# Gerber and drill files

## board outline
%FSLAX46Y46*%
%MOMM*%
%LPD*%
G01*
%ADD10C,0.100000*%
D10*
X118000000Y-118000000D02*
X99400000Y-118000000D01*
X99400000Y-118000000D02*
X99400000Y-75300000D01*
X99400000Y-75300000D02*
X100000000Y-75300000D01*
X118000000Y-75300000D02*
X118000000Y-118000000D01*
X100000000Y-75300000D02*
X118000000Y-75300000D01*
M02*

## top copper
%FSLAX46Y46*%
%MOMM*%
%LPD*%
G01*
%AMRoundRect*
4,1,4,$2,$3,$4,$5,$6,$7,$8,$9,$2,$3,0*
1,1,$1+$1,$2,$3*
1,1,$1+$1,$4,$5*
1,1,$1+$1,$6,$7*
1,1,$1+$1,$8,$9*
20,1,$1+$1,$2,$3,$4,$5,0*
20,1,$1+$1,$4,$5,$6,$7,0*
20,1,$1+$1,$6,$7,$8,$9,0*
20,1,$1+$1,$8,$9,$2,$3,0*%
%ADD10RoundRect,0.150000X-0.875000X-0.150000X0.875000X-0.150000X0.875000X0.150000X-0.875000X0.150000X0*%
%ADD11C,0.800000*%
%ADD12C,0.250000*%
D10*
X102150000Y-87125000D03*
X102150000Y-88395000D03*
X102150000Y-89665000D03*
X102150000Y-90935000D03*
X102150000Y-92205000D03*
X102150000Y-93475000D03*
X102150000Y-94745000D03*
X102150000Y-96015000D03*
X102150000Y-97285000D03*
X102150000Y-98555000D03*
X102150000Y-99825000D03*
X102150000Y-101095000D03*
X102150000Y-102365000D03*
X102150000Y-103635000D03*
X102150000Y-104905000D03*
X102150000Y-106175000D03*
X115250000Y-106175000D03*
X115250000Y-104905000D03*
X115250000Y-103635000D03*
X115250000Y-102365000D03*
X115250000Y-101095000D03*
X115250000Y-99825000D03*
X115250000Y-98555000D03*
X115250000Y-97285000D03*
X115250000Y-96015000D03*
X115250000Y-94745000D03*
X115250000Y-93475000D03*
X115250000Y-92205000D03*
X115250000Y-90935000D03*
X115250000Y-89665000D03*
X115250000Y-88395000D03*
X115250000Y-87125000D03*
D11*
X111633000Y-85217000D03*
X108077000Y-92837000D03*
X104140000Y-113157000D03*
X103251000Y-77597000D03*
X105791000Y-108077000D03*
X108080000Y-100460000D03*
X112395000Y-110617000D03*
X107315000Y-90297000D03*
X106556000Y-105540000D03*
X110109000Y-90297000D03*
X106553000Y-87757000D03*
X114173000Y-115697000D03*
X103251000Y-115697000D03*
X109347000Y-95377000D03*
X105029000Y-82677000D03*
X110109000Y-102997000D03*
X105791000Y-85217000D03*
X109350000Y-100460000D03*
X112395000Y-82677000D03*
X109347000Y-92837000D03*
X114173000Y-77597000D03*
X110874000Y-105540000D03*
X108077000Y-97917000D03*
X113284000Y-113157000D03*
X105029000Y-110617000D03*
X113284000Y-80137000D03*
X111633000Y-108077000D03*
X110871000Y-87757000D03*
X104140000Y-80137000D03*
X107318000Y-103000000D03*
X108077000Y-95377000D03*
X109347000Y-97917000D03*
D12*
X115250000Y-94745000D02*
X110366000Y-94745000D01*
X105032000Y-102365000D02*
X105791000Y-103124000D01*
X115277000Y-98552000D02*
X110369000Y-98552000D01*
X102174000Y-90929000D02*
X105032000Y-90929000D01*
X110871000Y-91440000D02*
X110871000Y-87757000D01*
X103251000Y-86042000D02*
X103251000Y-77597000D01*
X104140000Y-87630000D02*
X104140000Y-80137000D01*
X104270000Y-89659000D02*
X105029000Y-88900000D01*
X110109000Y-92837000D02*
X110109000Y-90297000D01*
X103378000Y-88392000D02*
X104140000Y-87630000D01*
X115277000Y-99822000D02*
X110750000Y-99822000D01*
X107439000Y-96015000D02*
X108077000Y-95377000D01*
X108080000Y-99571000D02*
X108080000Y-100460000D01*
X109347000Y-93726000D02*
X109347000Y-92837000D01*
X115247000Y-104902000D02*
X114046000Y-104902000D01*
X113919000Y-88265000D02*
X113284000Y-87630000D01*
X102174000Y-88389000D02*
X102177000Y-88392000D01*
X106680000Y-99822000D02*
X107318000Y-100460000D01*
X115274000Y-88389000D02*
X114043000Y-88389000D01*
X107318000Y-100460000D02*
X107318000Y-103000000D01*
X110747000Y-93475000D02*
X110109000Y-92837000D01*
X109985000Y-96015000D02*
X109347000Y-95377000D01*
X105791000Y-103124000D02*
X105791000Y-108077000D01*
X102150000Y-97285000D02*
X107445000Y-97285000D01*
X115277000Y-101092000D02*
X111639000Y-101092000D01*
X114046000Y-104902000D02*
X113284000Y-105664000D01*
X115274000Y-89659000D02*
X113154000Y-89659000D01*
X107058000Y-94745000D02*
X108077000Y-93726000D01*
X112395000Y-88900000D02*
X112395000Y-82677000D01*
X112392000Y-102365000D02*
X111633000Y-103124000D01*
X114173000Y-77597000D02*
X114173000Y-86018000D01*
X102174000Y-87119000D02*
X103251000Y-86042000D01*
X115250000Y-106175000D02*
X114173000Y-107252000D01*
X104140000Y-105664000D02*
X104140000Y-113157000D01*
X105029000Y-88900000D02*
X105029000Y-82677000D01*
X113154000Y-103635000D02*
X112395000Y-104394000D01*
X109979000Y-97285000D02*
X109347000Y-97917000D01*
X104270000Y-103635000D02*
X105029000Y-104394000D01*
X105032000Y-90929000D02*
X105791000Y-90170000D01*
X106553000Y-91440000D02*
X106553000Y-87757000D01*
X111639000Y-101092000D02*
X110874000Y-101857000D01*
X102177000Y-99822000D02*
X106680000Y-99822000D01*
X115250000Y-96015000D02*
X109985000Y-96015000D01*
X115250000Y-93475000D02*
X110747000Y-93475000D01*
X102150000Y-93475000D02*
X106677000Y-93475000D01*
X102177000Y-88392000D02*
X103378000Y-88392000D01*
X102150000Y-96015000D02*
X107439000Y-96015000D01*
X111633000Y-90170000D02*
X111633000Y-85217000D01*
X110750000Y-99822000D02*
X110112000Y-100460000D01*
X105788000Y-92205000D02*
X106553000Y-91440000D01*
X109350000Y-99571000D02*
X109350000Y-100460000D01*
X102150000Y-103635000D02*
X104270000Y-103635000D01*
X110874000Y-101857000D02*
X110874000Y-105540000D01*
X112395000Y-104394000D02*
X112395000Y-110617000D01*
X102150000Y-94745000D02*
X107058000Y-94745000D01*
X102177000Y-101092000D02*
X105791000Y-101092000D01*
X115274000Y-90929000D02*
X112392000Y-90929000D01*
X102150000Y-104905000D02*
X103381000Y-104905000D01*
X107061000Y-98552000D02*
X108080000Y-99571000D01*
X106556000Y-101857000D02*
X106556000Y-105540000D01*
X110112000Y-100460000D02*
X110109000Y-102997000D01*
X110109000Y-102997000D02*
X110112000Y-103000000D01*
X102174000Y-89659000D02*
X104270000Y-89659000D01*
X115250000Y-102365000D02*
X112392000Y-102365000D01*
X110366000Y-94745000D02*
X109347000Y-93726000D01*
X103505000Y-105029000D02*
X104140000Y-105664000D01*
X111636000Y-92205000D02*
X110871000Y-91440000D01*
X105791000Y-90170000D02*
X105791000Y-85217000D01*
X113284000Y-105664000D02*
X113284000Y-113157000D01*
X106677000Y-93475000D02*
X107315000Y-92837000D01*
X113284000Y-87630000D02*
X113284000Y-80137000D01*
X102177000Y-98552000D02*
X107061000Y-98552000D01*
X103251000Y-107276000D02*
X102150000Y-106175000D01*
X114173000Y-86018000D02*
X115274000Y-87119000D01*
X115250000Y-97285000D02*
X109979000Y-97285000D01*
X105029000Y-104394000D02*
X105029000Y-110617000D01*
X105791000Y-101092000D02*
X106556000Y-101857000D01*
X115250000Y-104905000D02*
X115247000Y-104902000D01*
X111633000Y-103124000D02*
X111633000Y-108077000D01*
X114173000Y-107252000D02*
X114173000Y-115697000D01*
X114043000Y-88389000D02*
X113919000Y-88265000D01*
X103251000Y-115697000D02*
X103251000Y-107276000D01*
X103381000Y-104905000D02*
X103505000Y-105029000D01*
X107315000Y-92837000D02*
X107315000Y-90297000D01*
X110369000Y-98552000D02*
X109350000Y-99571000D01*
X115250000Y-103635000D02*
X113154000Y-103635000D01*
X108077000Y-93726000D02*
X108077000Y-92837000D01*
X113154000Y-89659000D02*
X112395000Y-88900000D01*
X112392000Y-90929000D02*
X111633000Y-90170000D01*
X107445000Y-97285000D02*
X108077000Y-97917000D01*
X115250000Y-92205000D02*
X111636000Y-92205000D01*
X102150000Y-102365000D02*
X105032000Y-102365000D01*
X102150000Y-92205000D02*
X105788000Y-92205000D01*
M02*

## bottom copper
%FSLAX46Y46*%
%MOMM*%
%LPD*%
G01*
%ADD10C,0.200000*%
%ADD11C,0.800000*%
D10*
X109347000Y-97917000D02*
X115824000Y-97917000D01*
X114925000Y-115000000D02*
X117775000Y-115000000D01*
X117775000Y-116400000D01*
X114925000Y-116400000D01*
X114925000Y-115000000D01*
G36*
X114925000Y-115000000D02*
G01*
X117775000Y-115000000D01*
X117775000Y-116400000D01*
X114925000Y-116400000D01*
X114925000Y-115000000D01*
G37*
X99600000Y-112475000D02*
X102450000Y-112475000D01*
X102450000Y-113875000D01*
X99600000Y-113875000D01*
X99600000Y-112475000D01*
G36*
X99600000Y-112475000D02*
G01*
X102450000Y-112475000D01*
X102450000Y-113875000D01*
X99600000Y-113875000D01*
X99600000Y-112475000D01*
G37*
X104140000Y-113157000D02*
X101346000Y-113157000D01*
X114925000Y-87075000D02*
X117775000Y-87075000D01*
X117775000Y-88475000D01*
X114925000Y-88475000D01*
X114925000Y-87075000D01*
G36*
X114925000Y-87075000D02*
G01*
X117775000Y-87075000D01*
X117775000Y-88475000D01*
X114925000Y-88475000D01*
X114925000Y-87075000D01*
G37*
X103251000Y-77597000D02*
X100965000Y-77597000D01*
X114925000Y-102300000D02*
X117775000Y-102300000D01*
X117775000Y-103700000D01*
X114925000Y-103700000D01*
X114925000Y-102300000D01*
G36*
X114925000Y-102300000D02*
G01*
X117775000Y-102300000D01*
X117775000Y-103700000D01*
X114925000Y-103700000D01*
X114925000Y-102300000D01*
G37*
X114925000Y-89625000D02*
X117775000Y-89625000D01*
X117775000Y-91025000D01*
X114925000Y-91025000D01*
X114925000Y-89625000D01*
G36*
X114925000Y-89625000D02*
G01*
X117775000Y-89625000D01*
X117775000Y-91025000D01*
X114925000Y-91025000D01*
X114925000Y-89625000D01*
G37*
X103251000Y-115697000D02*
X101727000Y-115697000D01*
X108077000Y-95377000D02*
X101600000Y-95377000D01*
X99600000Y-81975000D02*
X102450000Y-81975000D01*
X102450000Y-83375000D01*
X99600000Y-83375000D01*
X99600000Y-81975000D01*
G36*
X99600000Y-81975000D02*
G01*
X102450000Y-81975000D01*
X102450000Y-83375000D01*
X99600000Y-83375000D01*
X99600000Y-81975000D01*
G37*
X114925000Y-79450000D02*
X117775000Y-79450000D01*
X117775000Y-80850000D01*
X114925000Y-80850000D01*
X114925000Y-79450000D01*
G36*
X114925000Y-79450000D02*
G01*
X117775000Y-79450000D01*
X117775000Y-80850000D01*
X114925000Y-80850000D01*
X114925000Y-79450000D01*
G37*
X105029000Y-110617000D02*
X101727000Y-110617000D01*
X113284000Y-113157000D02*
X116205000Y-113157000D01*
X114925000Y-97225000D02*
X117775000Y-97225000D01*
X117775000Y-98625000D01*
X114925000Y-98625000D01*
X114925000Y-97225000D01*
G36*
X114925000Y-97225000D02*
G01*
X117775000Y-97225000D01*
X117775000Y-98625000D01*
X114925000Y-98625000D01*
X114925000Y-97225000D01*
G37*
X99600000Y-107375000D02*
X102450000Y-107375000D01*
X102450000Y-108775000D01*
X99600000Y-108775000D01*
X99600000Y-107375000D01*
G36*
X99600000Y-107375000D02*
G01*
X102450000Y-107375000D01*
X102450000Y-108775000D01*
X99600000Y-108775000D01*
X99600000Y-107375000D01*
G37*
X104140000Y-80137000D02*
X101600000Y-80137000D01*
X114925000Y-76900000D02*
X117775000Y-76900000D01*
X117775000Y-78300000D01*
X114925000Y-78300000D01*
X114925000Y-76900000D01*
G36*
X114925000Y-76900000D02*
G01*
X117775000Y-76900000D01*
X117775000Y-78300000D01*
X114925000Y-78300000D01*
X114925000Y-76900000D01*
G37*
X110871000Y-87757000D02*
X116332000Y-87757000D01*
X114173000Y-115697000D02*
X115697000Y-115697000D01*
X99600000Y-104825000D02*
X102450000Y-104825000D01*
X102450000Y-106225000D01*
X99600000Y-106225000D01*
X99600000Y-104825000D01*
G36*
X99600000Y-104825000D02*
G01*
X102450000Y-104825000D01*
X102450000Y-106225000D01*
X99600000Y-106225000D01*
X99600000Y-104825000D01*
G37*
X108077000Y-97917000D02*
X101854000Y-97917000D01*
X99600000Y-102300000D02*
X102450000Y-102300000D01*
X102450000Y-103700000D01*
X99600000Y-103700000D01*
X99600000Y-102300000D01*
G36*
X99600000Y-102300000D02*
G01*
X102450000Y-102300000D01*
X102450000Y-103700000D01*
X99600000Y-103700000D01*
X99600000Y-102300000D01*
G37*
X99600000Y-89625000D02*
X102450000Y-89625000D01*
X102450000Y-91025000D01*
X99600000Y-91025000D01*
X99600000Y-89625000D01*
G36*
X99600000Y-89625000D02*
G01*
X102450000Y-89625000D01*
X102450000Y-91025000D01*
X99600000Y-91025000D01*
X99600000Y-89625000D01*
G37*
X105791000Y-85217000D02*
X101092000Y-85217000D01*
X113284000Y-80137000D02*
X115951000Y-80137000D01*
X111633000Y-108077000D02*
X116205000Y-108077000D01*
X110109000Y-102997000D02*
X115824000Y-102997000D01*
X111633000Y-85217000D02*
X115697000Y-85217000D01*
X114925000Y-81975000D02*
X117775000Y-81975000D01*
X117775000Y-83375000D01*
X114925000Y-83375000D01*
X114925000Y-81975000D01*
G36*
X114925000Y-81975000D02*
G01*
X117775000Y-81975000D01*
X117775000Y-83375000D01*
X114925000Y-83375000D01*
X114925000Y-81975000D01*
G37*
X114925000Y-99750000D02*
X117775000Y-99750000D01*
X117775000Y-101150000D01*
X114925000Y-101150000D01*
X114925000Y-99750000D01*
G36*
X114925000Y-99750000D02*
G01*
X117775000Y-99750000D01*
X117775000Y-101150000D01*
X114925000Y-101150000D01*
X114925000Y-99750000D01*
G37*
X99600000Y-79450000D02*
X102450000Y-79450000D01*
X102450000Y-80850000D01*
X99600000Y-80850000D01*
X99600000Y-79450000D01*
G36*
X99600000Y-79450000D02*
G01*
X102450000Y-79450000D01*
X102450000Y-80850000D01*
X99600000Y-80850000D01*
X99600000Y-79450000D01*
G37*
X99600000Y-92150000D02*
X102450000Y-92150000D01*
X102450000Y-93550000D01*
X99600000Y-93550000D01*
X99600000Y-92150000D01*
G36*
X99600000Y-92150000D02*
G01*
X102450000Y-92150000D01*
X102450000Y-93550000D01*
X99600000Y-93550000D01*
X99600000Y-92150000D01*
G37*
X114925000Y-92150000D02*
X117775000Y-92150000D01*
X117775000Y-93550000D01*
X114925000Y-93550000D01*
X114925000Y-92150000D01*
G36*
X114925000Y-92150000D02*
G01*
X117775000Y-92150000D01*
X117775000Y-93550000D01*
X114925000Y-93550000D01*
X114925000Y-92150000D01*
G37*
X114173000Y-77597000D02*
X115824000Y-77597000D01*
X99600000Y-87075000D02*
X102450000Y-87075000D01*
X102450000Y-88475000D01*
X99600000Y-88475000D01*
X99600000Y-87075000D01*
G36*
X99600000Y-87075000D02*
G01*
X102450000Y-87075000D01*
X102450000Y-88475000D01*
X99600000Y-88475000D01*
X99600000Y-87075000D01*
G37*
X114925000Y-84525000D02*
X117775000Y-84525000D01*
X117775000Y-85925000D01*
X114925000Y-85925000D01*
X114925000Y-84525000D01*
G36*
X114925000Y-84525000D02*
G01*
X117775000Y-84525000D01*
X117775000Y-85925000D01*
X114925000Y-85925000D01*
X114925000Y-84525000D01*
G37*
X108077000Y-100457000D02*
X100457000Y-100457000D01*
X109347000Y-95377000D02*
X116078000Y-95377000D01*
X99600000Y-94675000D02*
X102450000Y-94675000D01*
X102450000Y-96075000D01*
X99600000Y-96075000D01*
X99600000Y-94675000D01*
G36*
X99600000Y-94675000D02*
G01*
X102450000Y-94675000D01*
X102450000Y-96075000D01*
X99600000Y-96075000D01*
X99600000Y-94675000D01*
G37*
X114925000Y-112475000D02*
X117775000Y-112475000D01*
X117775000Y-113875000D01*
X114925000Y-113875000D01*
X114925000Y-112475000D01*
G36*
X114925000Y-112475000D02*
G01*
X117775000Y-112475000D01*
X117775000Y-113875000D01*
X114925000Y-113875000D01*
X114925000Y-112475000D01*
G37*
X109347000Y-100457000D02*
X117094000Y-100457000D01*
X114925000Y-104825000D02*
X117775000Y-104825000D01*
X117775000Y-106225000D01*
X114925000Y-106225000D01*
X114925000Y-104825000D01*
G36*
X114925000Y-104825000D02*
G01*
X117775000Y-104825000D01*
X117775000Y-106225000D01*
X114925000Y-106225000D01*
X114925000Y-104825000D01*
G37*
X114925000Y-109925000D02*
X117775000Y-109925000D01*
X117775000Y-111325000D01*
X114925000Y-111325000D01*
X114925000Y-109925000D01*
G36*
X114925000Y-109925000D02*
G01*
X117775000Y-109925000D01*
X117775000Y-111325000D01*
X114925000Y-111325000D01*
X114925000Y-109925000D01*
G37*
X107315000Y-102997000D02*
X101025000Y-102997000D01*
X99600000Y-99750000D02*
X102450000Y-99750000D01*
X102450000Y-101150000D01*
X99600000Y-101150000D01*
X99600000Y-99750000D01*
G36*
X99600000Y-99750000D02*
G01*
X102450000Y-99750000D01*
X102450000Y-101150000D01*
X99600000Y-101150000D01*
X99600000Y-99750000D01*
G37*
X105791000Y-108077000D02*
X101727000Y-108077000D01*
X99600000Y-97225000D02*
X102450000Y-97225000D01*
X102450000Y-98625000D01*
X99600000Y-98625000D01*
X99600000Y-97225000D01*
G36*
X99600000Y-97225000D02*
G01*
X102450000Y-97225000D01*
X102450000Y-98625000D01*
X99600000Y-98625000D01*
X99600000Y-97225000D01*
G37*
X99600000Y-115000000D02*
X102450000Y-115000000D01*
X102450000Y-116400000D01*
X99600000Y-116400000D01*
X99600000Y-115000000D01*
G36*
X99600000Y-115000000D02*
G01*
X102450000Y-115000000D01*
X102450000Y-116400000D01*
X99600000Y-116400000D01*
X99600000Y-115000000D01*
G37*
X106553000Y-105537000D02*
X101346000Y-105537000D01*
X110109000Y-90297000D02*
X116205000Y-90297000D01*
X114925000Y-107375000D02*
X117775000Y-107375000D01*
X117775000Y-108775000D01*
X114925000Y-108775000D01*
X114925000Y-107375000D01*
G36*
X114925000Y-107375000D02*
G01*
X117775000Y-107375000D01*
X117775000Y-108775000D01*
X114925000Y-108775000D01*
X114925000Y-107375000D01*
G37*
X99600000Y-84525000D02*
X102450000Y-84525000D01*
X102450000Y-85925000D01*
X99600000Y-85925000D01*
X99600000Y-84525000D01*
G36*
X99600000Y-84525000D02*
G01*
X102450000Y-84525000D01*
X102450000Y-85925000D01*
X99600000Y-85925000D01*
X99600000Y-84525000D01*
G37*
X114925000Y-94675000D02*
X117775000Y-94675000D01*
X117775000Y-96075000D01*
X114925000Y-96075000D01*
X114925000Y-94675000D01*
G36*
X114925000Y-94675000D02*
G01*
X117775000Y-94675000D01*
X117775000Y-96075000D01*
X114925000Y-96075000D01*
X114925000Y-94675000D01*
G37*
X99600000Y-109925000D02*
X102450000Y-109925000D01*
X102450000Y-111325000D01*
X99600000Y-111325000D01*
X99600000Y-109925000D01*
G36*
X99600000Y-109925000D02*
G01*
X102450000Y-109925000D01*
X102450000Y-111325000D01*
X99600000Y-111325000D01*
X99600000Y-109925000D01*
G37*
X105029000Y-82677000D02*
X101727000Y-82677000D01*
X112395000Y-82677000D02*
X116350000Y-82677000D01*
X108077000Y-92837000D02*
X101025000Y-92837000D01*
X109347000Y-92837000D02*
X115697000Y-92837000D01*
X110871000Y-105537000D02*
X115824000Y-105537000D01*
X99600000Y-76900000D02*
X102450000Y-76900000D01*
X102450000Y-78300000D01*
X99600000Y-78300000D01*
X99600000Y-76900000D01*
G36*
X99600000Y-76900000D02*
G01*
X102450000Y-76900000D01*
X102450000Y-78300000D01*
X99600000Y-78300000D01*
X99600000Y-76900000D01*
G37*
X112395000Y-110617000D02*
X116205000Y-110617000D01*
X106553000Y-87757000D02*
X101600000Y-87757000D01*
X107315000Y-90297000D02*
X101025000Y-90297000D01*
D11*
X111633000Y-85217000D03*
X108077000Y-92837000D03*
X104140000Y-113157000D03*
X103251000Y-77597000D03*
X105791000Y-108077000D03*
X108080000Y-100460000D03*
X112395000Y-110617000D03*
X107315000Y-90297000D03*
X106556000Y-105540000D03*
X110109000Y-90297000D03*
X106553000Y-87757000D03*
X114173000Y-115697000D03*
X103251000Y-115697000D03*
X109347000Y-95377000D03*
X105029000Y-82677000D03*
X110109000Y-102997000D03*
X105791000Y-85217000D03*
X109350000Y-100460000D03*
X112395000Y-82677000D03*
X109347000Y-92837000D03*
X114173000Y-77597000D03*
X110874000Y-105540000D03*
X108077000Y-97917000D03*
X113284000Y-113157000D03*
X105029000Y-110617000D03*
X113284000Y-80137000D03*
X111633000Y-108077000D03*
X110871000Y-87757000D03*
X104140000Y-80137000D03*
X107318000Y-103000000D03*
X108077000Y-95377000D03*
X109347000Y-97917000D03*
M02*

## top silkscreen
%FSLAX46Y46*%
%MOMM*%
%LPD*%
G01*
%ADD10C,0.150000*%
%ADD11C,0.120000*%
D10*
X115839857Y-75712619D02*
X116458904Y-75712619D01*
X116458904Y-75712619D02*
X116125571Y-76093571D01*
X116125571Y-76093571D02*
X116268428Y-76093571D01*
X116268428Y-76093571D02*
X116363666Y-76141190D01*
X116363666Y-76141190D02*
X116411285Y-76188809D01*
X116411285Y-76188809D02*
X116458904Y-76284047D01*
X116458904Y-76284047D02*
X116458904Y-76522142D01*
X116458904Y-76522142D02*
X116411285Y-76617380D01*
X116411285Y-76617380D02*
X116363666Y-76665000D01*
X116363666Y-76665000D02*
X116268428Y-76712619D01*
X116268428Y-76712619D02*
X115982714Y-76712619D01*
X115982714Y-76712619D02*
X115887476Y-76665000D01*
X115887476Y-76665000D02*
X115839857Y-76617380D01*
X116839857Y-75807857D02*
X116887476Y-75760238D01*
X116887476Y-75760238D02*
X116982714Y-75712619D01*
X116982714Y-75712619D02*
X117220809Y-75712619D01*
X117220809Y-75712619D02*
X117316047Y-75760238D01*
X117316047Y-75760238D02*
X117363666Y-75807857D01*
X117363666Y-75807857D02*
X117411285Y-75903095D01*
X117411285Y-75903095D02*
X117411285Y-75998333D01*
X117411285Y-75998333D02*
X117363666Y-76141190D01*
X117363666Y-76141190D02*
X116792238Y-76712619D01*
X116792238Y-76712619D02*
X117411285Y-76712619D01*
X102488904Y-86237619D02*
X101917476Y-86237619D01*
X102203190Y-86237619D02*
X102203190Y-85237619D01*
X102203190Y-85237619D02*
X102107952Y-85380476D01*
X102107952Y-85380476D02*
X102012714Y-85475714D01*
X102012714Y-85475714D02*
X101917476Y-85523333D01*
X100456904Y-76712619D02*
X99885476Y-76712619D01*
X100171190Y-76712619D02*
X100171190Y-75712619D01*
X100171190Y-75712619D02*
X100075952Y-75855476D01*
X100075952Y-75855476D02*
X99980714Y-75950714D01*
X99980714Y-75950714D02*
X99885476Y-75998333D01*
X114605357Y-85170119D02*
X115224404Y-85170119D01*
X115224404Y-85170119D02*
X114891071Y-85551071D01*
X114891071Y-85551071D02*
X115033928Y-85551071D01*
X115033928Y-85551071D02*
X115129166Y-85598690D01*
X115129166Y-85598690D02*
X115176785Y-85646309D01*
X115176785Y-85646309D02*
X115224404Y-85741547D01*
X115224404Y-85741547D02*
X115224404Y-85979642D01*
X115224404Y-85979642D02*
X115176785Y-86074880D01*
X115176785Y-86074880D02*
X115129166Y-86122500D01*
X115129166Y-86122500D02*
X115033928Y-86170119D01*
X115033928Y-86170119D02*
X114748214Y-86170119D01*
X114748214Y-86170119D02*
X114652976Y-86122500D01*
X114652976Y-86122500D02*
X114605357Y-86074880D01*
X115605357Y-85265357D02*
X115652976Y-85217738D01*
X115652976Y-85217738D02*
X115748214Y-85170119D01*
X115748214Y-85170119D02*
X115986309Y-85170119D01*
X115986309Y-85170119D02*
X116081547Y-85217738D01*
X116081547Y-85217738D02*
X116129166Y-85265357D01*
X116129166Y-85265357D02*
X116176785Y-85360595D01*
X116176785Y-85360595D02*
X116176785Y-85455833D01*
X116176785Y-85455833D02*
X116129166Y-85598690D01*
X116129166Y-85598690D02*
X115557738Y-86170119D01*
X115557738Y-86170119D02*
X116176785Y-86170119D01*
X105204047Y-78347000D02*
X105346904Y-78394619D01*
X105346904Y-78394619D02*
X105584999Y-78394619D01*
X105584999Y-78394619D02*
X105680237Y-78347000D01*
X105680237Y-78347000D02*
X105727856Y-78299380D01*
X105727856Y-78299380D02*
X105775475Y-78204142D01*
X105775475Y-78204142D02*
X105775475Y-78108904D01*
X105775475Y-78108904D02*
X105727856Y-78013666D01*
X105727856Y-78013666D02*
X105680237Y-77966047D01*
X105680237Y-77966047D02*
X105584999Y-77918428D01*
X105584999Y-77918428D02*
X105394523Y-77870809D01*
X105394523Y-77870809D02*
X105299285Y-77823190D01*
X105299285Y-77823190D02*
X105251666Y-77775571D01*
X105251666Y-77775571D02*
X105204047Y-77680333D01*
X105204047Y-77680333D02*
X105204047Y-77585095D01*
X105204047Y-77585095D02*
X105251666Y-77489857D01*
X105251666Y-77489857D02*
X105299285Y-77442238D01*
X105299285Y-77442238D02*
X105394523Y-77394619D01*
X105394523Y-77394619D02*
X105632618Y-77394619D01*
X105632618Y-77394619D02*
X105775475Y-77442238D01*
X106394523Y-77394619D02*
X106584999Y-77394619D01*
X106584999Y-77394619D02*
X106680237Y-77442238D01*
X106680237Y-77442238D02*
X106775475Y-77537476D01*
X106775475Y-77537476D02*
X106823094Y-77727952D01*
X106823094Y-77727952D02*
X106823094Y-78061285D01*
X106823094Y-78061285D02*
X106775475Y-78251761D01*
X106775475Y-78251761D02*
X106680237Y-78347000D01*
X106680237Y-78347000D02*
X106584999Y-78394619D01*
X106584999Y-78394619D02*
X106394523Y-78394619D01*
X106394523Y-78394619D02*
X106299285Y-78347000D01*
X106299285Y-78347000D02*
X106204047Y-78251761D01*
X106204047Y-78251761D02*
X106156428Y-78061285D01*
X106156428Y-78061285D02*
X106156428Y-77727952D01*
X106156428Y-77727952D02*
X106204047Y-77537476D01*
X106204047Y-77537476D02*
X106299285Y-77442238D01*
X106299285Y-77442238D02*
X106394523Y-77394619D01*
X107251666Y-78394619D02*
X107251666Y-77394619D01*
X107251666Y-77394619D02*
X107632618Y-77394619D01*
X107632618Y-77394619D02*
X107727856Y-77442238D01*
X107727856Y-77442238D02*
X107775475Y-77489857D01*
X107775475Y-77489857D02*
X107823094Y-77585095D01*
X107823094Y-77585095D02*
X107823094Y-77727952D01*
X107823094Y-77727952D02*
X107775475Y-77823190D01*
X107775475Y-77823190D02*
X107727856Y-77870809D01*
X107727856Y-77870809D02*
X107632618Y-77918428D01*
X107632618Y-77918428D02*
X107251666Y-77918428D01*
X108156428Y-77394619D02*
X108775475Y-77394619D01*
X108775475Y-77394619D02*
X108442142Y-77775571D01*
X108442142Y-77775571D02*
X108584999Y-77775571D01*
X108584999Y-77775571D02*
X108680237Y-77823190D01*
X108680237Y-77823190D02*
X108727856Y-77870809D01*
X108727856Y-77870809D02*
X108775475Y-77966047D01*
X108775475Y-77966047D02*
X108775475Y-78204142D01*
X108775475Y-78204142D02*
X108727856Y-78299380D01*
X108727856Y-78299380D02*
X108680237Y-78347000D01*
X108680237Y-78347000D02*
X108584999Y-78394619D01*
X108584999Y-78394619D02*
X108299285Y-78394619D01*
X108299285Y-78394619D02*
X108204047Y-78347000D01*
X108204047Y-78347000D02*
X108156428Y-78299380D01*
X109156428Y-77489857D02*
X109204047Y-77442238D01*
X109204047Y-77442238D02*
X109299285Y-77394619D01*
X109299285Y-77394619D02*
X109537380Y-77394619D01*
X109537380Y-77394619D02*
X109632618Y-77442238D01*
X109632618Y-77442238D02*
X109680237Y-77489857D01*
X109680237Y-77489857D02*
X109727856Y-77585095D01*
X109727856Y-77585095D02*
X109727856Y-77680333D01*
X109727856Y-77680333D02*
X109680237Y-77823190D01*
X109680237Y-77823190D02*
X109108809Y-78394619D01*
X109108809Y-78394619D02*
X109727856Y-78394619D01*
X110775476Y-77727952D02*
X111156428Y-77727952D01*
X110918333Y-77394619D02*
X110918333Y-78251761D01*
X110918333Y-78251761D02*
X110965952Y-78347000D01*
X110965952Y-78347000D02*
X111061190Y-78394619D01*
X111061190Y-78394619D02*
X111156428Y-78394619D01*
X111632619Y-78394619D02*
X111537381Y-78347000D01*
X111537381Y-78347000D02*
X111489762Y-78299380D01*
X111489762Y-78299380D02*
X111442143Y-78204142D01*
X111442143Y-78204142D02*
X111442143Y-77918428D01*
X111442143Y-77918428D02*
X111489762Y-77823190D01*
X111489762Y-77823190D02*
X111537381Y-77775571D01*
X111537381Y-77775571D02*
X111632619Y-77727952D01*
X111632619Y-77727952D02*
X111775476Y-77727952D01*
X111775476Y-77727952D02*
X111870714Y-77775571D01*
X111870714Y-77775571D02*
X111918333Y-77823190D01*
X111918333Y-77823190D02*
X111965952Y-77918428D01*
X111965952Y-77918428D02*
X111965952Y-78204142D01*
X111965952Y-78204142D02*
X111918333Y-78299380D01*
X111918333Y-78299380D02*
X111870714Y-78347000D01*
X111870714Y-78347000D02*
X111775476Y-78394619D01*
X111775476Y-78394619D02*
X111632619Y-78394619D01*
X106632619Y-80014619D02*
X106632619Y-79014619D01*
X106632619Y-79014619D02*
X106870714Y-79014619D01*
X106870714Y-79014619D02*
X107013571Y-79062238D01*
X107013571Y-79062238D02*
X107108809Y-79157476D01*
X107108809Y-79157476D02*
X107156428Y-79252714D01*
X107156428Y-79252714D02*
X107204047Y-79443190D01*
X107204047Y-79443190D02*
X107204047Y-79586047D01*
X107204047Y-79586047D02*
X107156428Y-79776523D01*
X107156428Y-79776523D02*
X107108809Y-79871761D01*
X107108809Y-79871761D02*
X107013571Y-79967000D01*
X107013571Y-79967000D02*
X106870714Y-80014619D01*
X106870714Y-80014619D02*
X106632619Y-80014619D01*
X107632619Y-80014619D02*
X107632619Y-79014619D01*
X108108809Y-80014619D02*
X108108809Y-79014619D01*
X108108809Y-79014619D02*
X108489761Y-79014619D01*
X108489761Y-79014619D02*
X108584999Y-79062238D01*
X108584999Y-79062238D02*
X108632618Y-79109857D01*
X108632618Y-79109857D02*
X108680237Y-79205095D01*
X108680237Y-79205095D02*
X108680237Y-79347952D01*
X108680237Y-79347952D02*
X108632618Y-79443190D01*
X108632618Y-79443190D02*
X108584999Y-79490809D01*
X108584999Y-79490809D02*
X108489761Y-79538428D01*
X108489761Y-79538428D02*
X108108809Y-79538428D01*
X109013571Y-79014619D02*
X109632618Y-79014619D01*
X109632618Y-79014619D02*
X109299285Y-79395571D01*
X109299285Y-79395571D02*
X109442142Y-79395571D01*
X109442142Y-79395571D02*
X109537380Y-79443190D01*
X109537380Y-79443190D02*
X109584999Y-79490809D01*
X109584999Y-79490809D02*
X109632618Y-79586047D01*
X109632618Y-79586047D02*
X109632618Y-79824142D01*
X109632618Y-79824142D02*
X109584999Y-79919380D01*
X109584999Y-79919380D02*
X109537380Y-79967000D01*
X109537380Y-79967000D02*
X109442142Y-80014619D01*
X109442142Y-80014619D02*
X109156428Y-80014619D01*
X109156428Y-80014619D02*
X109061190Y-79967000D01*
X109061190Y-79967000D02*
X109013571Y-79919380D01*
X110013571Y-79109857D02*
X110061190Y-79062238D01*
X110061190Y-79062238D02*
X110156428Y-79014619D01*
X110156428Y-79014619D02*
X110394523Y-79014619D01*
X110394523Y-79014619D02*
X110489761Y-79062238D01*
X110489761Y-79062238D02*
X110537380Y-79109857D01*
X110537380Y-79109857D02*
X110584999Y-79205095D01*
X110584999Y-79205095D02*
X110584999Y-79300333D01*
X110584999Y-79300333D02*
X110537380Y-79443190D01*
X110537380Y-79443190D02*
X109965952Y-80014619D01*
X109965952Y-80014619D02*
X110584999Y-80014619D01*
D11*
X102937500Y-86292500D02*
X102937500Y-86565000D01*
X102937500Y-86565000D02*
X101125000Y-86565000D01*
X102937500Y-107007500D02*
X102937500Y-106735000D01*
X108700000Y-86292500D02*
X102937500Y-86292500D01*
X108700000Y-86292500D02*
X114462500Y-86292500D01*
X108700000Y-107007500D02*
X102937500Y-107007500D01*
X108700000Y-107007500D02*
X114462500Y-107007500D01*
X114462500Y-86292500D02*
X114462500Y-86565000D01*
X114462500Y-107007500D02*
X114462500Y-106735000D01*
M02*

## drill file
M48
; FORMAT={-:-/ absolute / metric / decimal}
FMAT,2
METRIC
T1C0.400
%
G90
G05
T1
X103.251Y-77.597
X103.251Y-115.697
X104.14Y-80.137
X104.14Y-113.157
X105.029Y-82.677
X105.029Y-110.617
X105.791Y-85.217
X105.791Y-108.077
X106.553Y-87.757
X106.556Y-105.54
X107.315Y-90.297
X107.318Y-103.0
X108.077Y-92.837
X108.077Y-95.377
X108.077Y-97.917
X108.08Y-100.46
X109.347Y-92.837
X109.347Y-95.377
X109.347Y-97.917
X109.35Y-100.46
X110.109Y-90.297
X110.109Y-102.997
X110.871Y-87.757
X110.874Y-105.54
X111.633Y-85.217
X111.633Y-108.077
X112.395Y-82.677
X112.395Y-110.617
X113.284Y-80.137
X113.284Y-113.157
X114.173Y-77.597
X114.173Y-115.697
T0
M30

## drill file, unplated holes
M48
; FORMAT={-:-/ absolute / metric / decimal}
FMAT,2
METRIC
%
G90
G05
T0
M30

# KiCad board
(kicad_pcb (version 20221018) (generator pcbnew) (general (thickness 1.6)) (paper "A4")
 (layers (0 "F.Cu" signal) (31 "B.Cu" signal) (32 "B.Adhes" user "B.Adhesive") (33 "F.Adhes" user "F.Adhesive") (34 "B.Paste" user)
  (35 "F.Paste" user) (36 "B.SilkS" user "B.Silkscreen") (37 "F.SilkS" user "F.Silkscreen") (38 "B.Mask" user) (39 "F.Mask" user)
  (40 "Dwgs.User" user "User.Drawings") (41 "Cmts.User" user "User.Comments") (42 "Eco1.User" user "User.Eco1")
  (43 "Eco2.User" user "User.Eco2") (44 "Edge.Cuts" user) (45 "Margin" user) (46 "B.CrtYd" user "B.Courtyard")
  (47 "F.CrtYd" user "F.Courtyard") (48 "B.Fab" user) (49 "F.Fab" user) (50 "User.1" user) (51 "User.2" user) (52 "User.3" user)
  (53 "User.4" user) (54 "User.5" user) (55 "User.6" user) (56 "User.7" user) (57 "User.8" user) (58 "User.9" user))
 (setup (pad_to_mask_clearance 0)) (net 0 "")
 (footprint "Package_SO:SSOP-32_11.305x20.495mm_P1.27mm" (layer "F.Cu") (at 108.7 96.65)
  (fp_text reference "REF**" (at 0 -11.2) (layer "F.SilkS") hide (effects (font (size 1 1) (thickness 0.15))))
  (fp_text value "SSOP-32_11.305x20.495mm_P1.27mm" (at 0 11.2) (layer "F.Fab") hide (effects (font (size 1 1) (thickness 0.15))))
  (fp_line (start -5.7625 -10.3575) (end -5.7625 -10.085) (stroke (width 0.12) (type solid)) (layer "F.SilkS"))
  (fp_line (start -5.7625 -10.085) (end -7.575 -10.085) (stroke (width 0.12) (type solid)) (layer "F.SilkS"))
  (fp_line (start -5.7625 10.3575) (end -5.7625 10.085) (stroke (width 0.12) (type solid)) (layer "F.SilkS"))
  (fp_line (start 0 -10.3575) (end -5.7625 -10.3575) (stroke (width 0.12) (type solid)) (layer "F.SilkS"))
  (fp_line (start 0 -10.3575) (end 5.7625 -10.3575) (stroke (width 0.12) (type solid)) (layer "F.SilkS"))
  (fp_line (start 0 10.3575) (end -5.7625 10.3575) (stroke (width 0.12) (type solid)) (layer "F.SilkS"))
  (fp_line (start 0 10.3575) (end 5.7625 10.3575) (stroke (width 0.12) (type solid)) (layer "F.SilkS"))
  (fp_line (start 5.7625 -10.3575) (end 5.7625 -10.085) (stroke (width 0.12) (type solid)) (layer "F.SilkS"))
  (fp_line (start 5.7625 10.3575) (end 5.7625 10.085) (stroke (width 0.12) (type solid)) (layer "F.SilkS"))
  (pad "1" smd roundrect (at -6.55 -9.525) (size 2.05 0.6) (layers "F.Cu" "F.Paste" "F.Mask") (roundrect_rratio 0.25))
  (pad "2" smd roundrect (at -6.55 -8.255) (size 2.05 0.6) (layers "F.Cu" "F.Paste" "F.Mask") (roundrect_rratio 0.25))
  (pad "3" smd roundrect (at -6.55 -6.985) (size 2.05 0.6) (layers "F.Cu" "F.Paste" "F.Mask") (roundrect_rratio 0.25))
  (pad "4" smd roundrect (at -6.55 -5.715) (size 2.05 0.6) (layers "F.Cu" "F.Paste" "F.Mask") (roundrect_rratio 0.25))
  (pad "5" smd roundrect (at -6.55 -4.445) (size 2.05 0.6) (layers "F.Cu" "F.Paste" "F.Mask") (roundrect_rratio 0.25))
  (pad "6" smd roundrect (at -6.55 -3.175) (size 2.05 0.6) (layers "F.Cu" "F.Paste" "F.Mask") (roundrect_rratio 0.25))
  (pad "7" smd roundrect (at -6.55 -1.905) (size 2.05 0.6) (layers "F.Cu" "F.Paste" "F.Mask") (roundrect_rratio 0.25))
  (pad "8" smd roundrect (at -6.55 -0.635) (size 2.05 0.6) (layers "F.Cu" "F.Paste" "F.Mask") (roundrect_rratio 0.25))
  (pad "9" smd roundrect (at -6.55 0.635) (size 2.05 0.6) (layers "F.Cu" "F.Paste" "F.Mask") (roundrect_rratio 0.25))
  (pad "10" smd roundrect (at -6.55 1.905) (size 2.05 0.6) (layers "F.Cu" "F.Paste" "F.Mask") (roundrect_rratio 0.25))
  (pad "11" smd roundrect (at -6.55 3.175) (size 2.05 0.6) (layers "F.Cu" "F.Paste" "F.Mask") (roundrect_rratio 0.25))
  (pad "12" smd roundrect (at -6.55 4.445) (size 2.05 0.6) (layers "F.Cu" "F.Paste" "F.Mask") (roundrect_rratio 0.25))
  (pad "13" smd roundrect (at -6.55 5.715) (size 2.05 0.6) (layers "F.Cu" "F.Paste" "F.Mask") (roundrect_rratio 0.25))
  (pad "14" smd roundrect (at -6.55 6.985) (size 2.05 0.6) (layers "F.Cu" "F.Paste" "F.Mask") (roundrect_rratio 0.25))
  (pad "15" smd roundrect (at -6.55 8.255) (size 2.05 0.6) (layers "F.Cu" "F.Paste" "F.Mask") (roundrect_rratio 0.25))
  (pad "16" smd roundrect (at -6.55 9.525) (size 2.05 0.6) (layers "F.Cu" "F.Paste" "F.Mask") (roundrect_rratio 0.25))
  (pad "17" smd roundrect (at 6.55 9.525) (size 2.05 0.6) (layers "F.Cu" "F.Paste" "F.Mask") (roundrect_rratio 0.25))
  (pad "18" smd roundrect (at 6.55 8.255) (size 2.05 0.6) (layers "F.Cu" "F.Paste" "F.Mask") (roundrect_rratio 0.25))
  (pad "19" smd roundrect (at 6.55 6.985) (size 2.05 0.6) (layers "F.Cu" "F.Paste" "F.Mask") (roundrect_rratio 0.25))
  (pad "20" smd roundrect (at 6.55 5.715) (size 2.05 0.6) (layers "F.Cu" "F.Paste" "F.Mask") (roundrect_rratio 0.25))
  (pad "21" smd roundrect (at 6.55 4.445) (size 2.05 0.6) (layers "F.Cu" "F.Paste" "F.Mask") (roundrect_rratio 0.25))
  (pad "22" smd roundrect (at 6.55 3.175) (size 2.05 0.6) (layers "F.Cu" "F.Paste" "F.Mask") (roundrect_rratio 0.25))
  (pad "23" smd roundrect (at 6.55 1.905) (size 2.05 0.6) (layers "F.Cu" "F.Paste" "F.Mask") (roundrect_rratio 0.25))
  (pad "24" smd roundrect (at 6.55 0.635) (size 2.05 0.6) (layers "F.Cu" "F.Paste" "F.Mask") (roundrect_rratio 0.25))
  (pad "25" smd roundrect (at 6.55 -0.635) (size 2.05 0.6) (layers "F.Cu" "F.Paste" "F.Mask") (roundrect_rratio 0.25))
  (pad "26" smd roundrect (at 6.55 -1.905) (size 2.05 0.6) (layers "F.Cu" "F.Paste" "F.Mask") (roundrect_rratio 0.25))
  (pad "27" smd roundrect (at 6.55 -3.175) (size 2.05 0.6) (layers "F.Cu" "F.Paste" "F.Mask") (roundrect_rratio 0.25))
  (pad "28" smd roundrect (at 6.55 -4.445) (size 2.05 0.6) (layers "F.Cu" "F.Paste" "F.Mask") (roundrect_rratio 0.25))
  (pad "29" smd roundrect (at 6.55 -5.715) (size 2.05 0.6) (layers "F.Cu" "F.Paste" "F.Mask") (roundrect_rratio 0.25))
  (pad "30" smd roundrect (at 6.55 -6.985) (size 2.05 0.6) (layers "F.Cu" "F.Paste" "F.Mask") (roundrect_rratio 0.25))
  (pad "31" smd roundrect (at 6.55 -8.255) (size 2.05 0.6) (layers "F.Cu" "F.Paste" "F.Mask") (roundrect_rratio 0.25))
  (pad "32" smd roundrect (at 6.55 -9.525) (size 2.05 0.6) (layers "F.Cu" "F.Paste" "F.Mask") (roundrect_rratio 0.25)))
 (gr_line (start 109.347 97.917) (end 115.824 97.917) (stroke (width 0.2) (type default)) (layer "B.Cu"))
 (gr_rect (start 114.925 115) (end 117.775 116.4) (stroke (width 0.2) (type solid)) (fill solid) (layer "B.Cu"))
 (gr_rect (start 99.6 112.475) (end 102.45 113.875) (stroke (width 0.2) (type solid)) (fill solid) (layer "B.Cu"))
 (gr_line (start 104.14 113.157) (end 101.346 113.157) (stroke (width 0.2) (type default)) (layer "B.Cu"))
 (gr_rect (start 114.925 87.075) (end 117.775 88.475) (stroke (width 0.2) (type solid)) (fill solid) (layer "B.Cu"))
 (gr_line (start 103.251 77.597) (end 100.965 77.597) (stroke (width 0.2) (type default)) (layer "B.Cu"))
 (gr_rect (start 114.925 102.3) (end 117.775 103.7) (stroke (width 0.2) (type solid)) (fill solid) (layer "B.Cu"))
 (gr_rect (start 114.925 89.625) (end 117.775 91.025) (stroke (width 0.2) (type solid)) (fill solid) (layer "B.Cu"))
 (gr_line (start 103.251 115.697) (end 101.727 115.697) (stroke (width 0.2) (type default)) (layer "B.Cu"))
 (gr_line (start 108.077 95.377) (end 101.6 95.377) (stroke (width 0.2) (type default)) (layer "B.Cu"))
 (gr_rect (start 99.6 81.975) (end 102.45 83.375) (stroke (width 0.2) (type solid)) (fill solid) (layer "B.Cu"))
 (gr_rect (start 114.925 79.45) (end 117.775 80.85) (stroke (width 0.2) (type solid)) (fill solid) (layer "B.Cu"))
 (gr_line (start 105.029 110.617) (end 101.727 110.617) (stroke (width 0.2) (type default)) (layer "B.Cu"))
 (gr_line (start 113.284 113.157) (end 116.205 113.157) (stroke (width 0.2) (type default)) (layer "B.Cu"))
 (gr_rect (start 114.925 97.225) (end 117.775 98.625) (stroke (width 0.2) (type solid)) (fill solid) (layer "B.Cu"))
 (gr_rect (start 99.6 107.375) (end 102.45 108.775) (stroke (width 0.2) (type solid)) (fill solid) (layer "B.Cu"))
 (gr_line (start 104.14 80.137) (end 101.6 80.137) (stroke (width 0.2) (type default)) (layer "B.Cu"))
 (gr_rect (start 114.925 76.9) (end 117.775 78.3) (stroke (width 0.2) (type solid)) (fill solid) (layer "B.Cu"))
 (gr_line (start 110.871 87.757) (end 116.332 87.757) (stroke (width 0.2) (type default)) (layer "B.Cu"))
 (gr_line (start 114.173 115.697) (end 115.697 115.697) (stroke (width 0.2) (type default)) (layer "B.Cu"))
 (gr_rect (start 99.6 104.825) (end 102.45 106.225) (stroke (width 0.2) (type solid)) (fill solid) (layer "B.Cu"))
 (gr_line (start 108.077 97.917) (end 101.854 97.917) (stroke (width 0.2) (type default)) (layer "B.Cu"))
 (gr_rect (start 99.6 102.3) (end 102.45 103.7) (stroke (width 0.2) (type solid)) (fill solid) (layer "B.Cu"))
 (gr_rect (start 99.6 89.625) (end 102.45 91.025) (stroke (width 0.2) (type solid)) (fill solid) (layer "B.Cu"))
 (gr_line (start 105.791 85.217) (end 101.092 85.217) (stroke (width 0.2) (type default)) (layer "B.Cu"))
 (gr_line (start 113.284 80.137) (end 115.951 80.137) (stroke (width 0.2) (type default)) (layer "B.Cu"))
 (gr_line (start 111.633 108.077) (end 116.205 108.077) (stroke (width 0.2) (type default)) (layer "B.Cu"))
 (gr_line (start 110.109 102.997) (end 115.824 102.997) (stroke (width 0.2) (type default)) (layer "B.Cu"))
 (gr_line (start 111.633 85.217) (end 115.697 85.217) (stroke (width 0.2) (type default)) (layer "B.Cu"))
 (gr_rect (start 114.925 81.975) (end 117.775 83.375) (stroke (width 0.2) (type solid)) (fill solid) (layer "B.Cu"))
 (gr_rect (start 114.925 99.75) (end 117.775 101.15) (stroke (width 0.2) (type solid)) (fill solid) (layer "B.Cu"))
 (gr_rect (start 99.6 79.45) (end 102.45 80.85) (stroke (width 0.2) (type solid)) (fill solid) (layer "B.Cu"))
 (gr_rect (start 99.6 92.15) (end 102.45 93.55) (stroke (width 0.2) (type solid)) (fill solid) (layer "B.Cu"))
 (gr_rect (start 114.925 92.15) (end 117.775 93.55) (stroke (width 0.2) (type solid)) (fill solid) (layer "B.Cu"))
 (gr_line (start 114.173 77.597) (end 115.824 77.597) (stroke (width 0.2) (type default)) (layer "B.Cu"))
 (gr_rect (start 99.6 87.075) (end 102.45 88.475) (stroke (width 0.2) (type solid)) (fill solid) (layer "B.Cu"))
 (gr_rect (start 114.925 84.525) (end 117.775 85.925) (stroke (width 0.2) (type solid)) (fill solid) (layer "B.Cu"))
 (gr_line (start 108.077 100.457) (end 100.457 100.457) (stroke (width 0.2) (type default)) (layer "B.Cu"))
 (gr_line (start 109.347 95.377) (end 116.078 95.377) (stroke (width 0.2) (type default)) (layer "B.Cu"))
 (gr_rect (start 99.6 94.675) (end 102.45 96.075) (stroke (width 0.2) (type solid)) (fill solid) (layer "B.Cu"))
 (gr_rect (start 114.925 112.475) (end 117.775 113.875) (stroke (width 0.2) (type solid)) (fill solid) (layer "B.Cu"))
 (gr_line (start 109.347 100.457) (end 117.094 100.457) (stroke (width 0.2) (type default)) (layer "B.Cu"))
 (gr_rect (start 114.925 104.825) (end 117.775 106.225) (stroke (width 0.2) (type solid)) (fill solid) (layer "B.Cu"))
 (gr_rect (start 114.925 109.925) (end 117.775 111.325) (stroke (width 0.2) (type solid)) (fill solid) (layer "B.Cu"))
 (gr_line (start 107.315 102.997) (end 101.025 102.997) (stroke (width 0.2) (type default)) (layer "B.Cu"))
 (gr_rect (start 99.6 99.75) (end 102.45 101.15) (stroke (width 0.2) (type solid)) (fill solid) (layer "B.Cu"))
 (gr_line (start 105.791 108.077) (end 101.727 108.077) (stroke (width 0.2) (type default)) (layer "B.Cu"))
 (gr_rect (start 99.6 97.225) (end 102.45 98.625) (stroke (width 0.2) (type solid)) (fill solid) (layer "B.Cu"))
 (gr_rect (start 99.6 115) (end 102.45 116.4) (stroke (width 0.2) (type solid)) (fill solid) (layer "B.Cu"))
 (gr_line (start 106.553 105.537) (end 101.346 105.537) (stroke (width 0.2) (type default)) (layer "B.Cu"))
 (gr_line (start 110.109 90.297) (end 116.205 90.297) (stroke (width 0.2) (type default)) (layer "B.Cu"))
 (gr_rect (start 114.925 107.375) (end 117.775 108.775) (stroke (width 0.2) (type solid)) (fill solid) (layer "B.Cu"))
 (gr_rect (start 99.6 84.525) (end 102.45 85.925) (stroke (width 0.2) (type solid)) (fill solid) (layer "B.Cu"))
 (gr_rect (start 114.925 94.675) (end 117.775 96.075) (stroke (width 0.2) (type solid)) (fill solid) (layer "B.Cu"))
 (gr_rect (start 99.6 109.925) (end 102.45 111.325) (stroke (width 0.2) (type solid)) (fill solid) (layer "B.Cu"))
 (gr_line (start 105.029 82.677) (end 101.727 82.677) (stroke (width 0.2) (type default)) (layer "B.Cu"))
 (gr_line (start 112.395 82.677) (end 116.35 82.677) (stroke (width 0.2) (type default)) (layer "B.Cu"))
 (gr_line (start 108.077 92.837) (end 101.025 92.837) (stroke (width 0.2) (type default)) (layer "B.Cu"))
 (gr_line (start 109.347 92.837) (end 115.697 92.837) (stroke (width 0.2) (type default)) (layer "B.Cu"))
 (gr_line (start 110.871 105.537) (end 115.824 105.537) (stroke (width 0.2) (type default)) (layer "B.Cu"))
 (gr_rect (start 99.6 76.9) (end 102.45 78.3) (stroke (width 0.2) (type solid)) (fill solid) (layer "B.Cu"))
 (gr_line (start 112.395 110.617) (end 116.205 110.617) (stroke (width 0.2) (type default)) (layer "B.Cu"))
 (gr_line (start 106.553 87.757) (end 101.6 87.757) (stroke (width 0.2) (type default)) (layer "B.Cu"))
 (gr_line (start 107.315 90.297) (end 101.025 90.297) (stroke (width 0.2) (type default)) (layer "B.Cu"))
 (gr_line (start 118 118) (end 99.4 118) (stroke (width 0.1) (type default)) (layer "Edge.Cuts"))
 (gr_line (start 99.4 118) (end 99.4 75.3) (stroke (width 0.1) (type default)) (layer "Edge.Cuts"))
 (gr_line (start 99.4 75.3) (end 100 75.3) (stroke (width 0.1) (type default)) (layer "Edge.Cuts"))
 (gr_line (start 118 75.3) (end 118 118) (stroke (width 0.1) (type default)) (layer "Edge.Cuts"))
 (gr_line (start 100 75.3) (end 118 75.3) (stroke (width 0.1) (type default)) (layer "Edge.Cuts"))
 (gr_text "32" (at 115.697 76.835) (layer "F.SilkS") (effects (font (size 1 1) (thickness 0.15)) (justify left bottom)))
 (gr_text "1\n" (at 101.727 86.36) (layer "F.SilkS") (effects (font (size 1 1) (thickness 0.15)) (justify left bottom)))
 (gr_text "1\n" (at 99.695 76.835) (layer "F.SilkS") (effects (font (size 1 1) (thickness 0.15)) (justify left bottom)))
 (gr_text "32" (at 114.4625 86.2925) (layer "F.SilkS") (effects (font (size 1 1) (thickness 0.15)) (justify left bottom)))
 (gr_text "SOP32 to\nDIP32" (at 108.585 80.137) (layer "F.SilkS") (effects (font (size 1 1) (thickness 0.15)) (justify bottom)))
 (segment (start 115.25 94.745) (end 110.366 94.745) (width 0.25) (layer "F.Cu") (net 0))
 (segment (start 105.032 102.365) (end 105.791 103.124) (width 0.25) (layer "F.Cu") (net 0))
 (segment (start 115.277 98.552) (end 110.369 98.552) (width 0.25) (layer "F.Cu") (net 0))
 (segment (start 102.174 90.929) (end 105.032 90.929) (width 0.25) (layer "F.Cu") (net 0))
 (segment (start 110.871 91.44) (end 110.871 87.757) (width 0.25) (layer "F.Cu") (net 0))
 (segment (start 103.251 86.042) (end 103.251 77.597) (width 0.25) (layer "F.Cu") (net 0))
 (segment (start 104.14 87.63) (end 104.14 80.137) (width 0.25) (layer "F.Cu") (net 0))
 (segment (start 104.27 89.659) (end 105.029 88.9) (width 0.25) (layer "F.Cu") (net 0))
 (segment (start 110.109 92.837) (end 110.109 90.297) (width 0.25) (layer "F.Cu") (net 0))
 (segment (start 103.378 88.392) (end 104.14 87.63) (width 0.25) (layer "F.Cu") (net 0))
 (segment (start 115.277 99.822) (end 110.75 99.822) (width 0.25) (layer "F.Cu") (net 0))
 (segment (start 107.439 96.015) (end 108.077 95.377) (width 0.25) (layer "F.Cu") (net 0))
 (segment (start 108.08 99.571) (end 108.08 100.46) (width 0.25) (layer "F.Cu") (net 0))
 (segment (start 109.347 93.726) (end 109.347 92.837) (width 0.25) (layer "F.Cu") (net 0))
 (segment (start 115.247 104.902) (end 114.046 104.902) (width 0.25) (layer "F.Cu") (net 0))
 (segment (start 113.919 88.265) (end 113.284 87.63) (width 0.25) (layer "F.Cu") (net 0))
 (segment (start 102.174 88.389) (end 102.177 88.392) (width 0.25) (layer "F.Cu") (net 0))
 (segment (start 106.68 99.822) (end 107.318 100.46) (width 0.25) (layer "F.Cu") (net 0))
 (segment (start 115.274 88.389) (end 114.043 88.389) (width 0.25) (layer "F.Cu") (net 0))
 (segment (start 107.318 100.46) (end 107.318 103) (width 0.25) (layer "F.Cu") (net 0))
 (segment (start 110.747 93.475) (end 110.109 92.837) (width 0.25) (layer "F.Cu") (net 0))
 (segment (start 109.985 96.015) (end 109.347 95.377) (width 0.25) (layer "F.Cu") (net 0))
 (segment (start 105.791 103.124) (end 105.791 108.077) (width 0.25) (layer "F.Cu") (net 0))
 (segment (start 102.15 97.285) (end 107.445 97.285) (width 0.25) (layer "F.Cu") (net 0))
 (segment (start 115.277 101.092) (end 111.639 101.092) (width 0.25) (layer "F.Cu") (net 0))
 (segment (start 114.046 104.902) (end 113.284 105.664) (width 0.25) (layer "F.Cu") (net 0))
 (segment (start 115.274 89.659) (end 113.154 89.659) (width 0.25) (layer "F.Cu") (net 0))
 (segment (start 107.058 94.745) (end 108.077 93.726) (width 0.25) (layer "F.Cu") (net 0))
 (segment (start 112.395 88.9) (end 112.395 82.677) (width 0.25) (layer "F.Cu") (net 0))
 (segment (start 112.392 102.365) (end 111.633 103.124) (width 0.25) (layer "F.Cu") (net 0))
 (segment (start 114.173 77.597) (end 114.173 86.018) (width 0.25) (layer "F.Cu") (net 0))
 (segment (start 102.174 87.119) (end 103.251 86.042) (width 0.25) (layer "F.Cu") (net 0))
 (segment (start 115.25 106.175) (end 114.173 107.252) (width 0.25) (layer "F.Cu") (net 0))
 (segment (start 104.14 105.664) (end 104.14 113.157) (width 0.25) (layer "F.Cu") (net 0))
 (segment (start 105.029 88.9) (end 105.029 82.677) (width 0.25) (layer "F.Cu") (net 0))
 (segment (start 113.154 103.635) (end 112.395 104.394) (width 0.25) (layer "F.Cu") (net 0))
 (segment (start 109.979 97.285) (end 109.347 97.917) (width 0.25) (layer "F.Cu") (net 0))
 (segment (start 104.27 103.635) (end 105.029 104.394) (width 0.25) (layer "F.Cu") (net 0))
 (segment (start 105.032 90.929) (end 105.791 90.17) (width 0.25) (layer "F.Cu") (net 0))
 (segment (start 106.553 91.44) (end 106.553 87.757) (width 0.25) (layer "F.Cu") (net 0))
 (segment (start 111.639 101.092) (end 110.874 101.857) (width 0.25) (layer "F.Cu") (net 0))
 (segment (start 102.177 99.822) (end 106.68 99.822) (width 0.25) (layer "F.Cu") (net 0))
 (segment (start 115.25 96.015) (end 109.985 96.015) (width 0.25) (layer "F.Cu") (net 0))
 (segment (start 115.25 93.475) (end 110.747 93.475) (width 0.25) (layer "F.Cu") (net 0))
 (segment (start 102.15 93.475) (end 106.677 93.475) (width 0.25) (layer "F.Cu") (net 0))
 (segment (start 102.177 88.392) (end 103.378 88.392) (width 0.25) (layer "F.Cu") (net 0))
 (segment (start 102.15 96.015) (end 107.439 96.015) (width 0.25) (layer "F.Cu") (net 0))
 (segment (start 111.633 90.17) (end 111.633 85.217) (width 0.25) (layer "F.Cu") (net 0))
 (segment (start 110.75 99.822) (end 110.112 100.46) (width 0.25) (layer "F.Cu") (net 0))
 (segment (start 105.788 92.205) (end 106.553 91.44) (width 0.25) (layer "F.Cu") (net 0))
 (segment (start 109.35 99.571) (end 109.35 100.46) (width 0.25) (layer "F.Cu") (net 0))
 (segment (start 102.15 103.635) (end 104.27 103.635) (width 0.25) (layer "F.Cu") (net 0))
 (segment (start 110.874 101.857) (end 110.874 105.54) (width 0.25) (layer "F.Cu") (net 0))
 (segment (start 112.395 104.394) (end 112.395 110.617) (width 0.25) (layer "F.Cu") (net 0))
 (segment (start 102.15 94.745) (end 107.058 94.745) (width 0.25) (layer "F.Cu") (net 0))
 (segment (start 102.177 101.092) (end 105.791 101.092) (width 0.25) (layer "F.Cu") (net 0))
 (segment (start 115.274 90.929) (end 112.392 90.929) (width 0.25) (layer "F.Cu") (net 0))
 (segment (start 102.15 104.905) (end 103.381 104.905) (width 0.25) (layer "F.Cu") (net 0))
 (segment (start 107.061 98.552) (end 108.08 99.571) (width 0.25) (layer "F.Cu") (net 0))
 (segment (start 106.556 101.857) (end 106.556 105.54) (width 0.25) (layer "F.Cu") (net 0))
 (segment (start 110.112 100.46) (end 110.109 102.997) (width 0.25) (layer "F.Cu") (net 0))
 (segment (start 110.109 102.997) (end 110.112 103) (width 0.25) (layer "F.Cu") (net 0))
 (segment (start 102.174 89.659) (end 104.27 89.659) (width 0.25) (layer "F.Cu") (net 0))
 (segment (start 115.25 102.365) (end 112.392 102.365) (width 0.25) (layer "F.Cu") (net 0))
 (segment (start 110.366 94.745) (end 109.347 93.726) (width 0.25) (layer "F.Cu") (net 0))
 (segment (start 103.505 105.029) (end 104.14 105.664) (width 0.25) (layer "F.Cu") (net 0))
 (segment (start 111.636 92.205) (end 110.871 91.44) (width 0.25) (layer "F.Cu") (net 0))
 (segment (start 105.791 90.17) (end 105.791 85.217) (width 0.25) (layer "F.Cu") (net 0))
 (segment (start 113.284 105.664) (end 113.284 113.157) (width 0.25) (layer "F.Cu") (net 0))
 (segment (start 106.677 93.475) (end 107.315 92.837) (width 0.25) (layer "F.Cu") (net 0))
 (segment (start 113.284 87.63) (end 113.284 80.137) (width 0.25) (layer "F.Cu") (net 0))
 (segment (start 102.177 98.552) (end 107.061 98.552) (width 0.25) (layer "F.Cu") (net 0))
 (segment (start 103.251 107.276) (end 102.15 106.175) (width 0.25) (layer "F.Cu") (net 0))
 (segment (start 114.173 86.018) (end 115.274 87.119) (width 0.25) (layer "F.Cu") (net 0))
 (segment (start 115.25 97.285) (end 109.979 97.285) (width 0.25) (layer "F.Cu") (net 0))
 (segment (start 105.029 104.394) (end 105.029 110.617) (width 0.25) (layer "F.Cu") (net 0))
 (segment (start 105.791 101.092) (end 106.556 101.857) (width 0.25) (layer "F.Cu") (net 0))
 (segment (start 115.25 104.905) (end 115.247 104.902) (width 0.25) (layer "F.Cu") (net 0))
 (segment (start 111.633 103.124) (end 111.633 108.077) (width 0.25) (layer "F.Cu") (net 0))
 (segment (start 114.173 107.252) (end 114.173 115.697) (width 0.25) (layer "F.Cu") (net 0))
 (segment (start 114.043 88.389) (end 113.919 88.265) (width 0.25) (layer "F.Cu") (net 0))
 (segment (start 103.251 115.697) (end 103.251 107.276) (width 0.25) (layer "F.Cu") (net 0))
 (segment (start 103.381 104.905) (end 103.505 105.029) (width 0.25) (layer "F.Cu") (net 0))
 (segment (start 107.315 92.837) (end 107.315 90.297) (width 0.25) (layer "F.Cu") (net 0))
 (segment (start 110.369 98.552) (end 109.35 99.571) (width 0.25) (layer "F.Cu") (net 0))
 (segment (start 115.25 103.635) (end 113.154 103.635) (width 0.25) (layer "F.Cu") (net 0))
 (segment (start 108.077 93.726) (end 108.077 92.837) (width 0.25) (layer "F.Cu") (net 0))
 (segment (start 113.154 89.659) (end 112.395 88.9) (width 0.25) (layer "F.Cu") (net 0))
 (segment (start 112.392 90.929) (end 111.633 90.17) (width 0.25) (layer "F.Cu") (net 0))
 (segment (start 107.445 97.285) (end 108.077 97.917) (width 0.25) (layer "F.Cu") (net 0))
 (segment (start 115.25 92.205) (end 111.636 92.205) (width 0.25) (layer "F.Cu") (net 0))
 (segment (start 102.15 102.365) (end 105.032 102.365) (width 0.25) (layer "F.Cu") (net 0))
 (segment (start 102.15 92.205) (end 105.788 92.205) (width 0.25) (layer "F.Cu") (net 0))
 (via (at 111.633 85.217) (size 0.8) (drill 0.4) (layers "F.Cu" "B.Cu") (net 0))
 (via (at 108.077 92.837) (size 0.8) (drill 0.4) (layers "F.Cu" "B.Cu") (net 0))
 (via (at 104.14 113.157) (size 0.8) (drill 0.4) (layers "F.Cu" "B.Cu") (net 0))
 (via (at 103.251 77.597) (size 0.8) (drill 0.4) (layers "F.Cu" "B.Cu") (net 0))
 (via (at 105.791 108.077) (size 0.8) (drill 0.4) (layers "F.Cu" "B.Cu") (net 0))
 (via (at 108.08 100.46) (size 0.8) (drill 0.4) (layers "F.Cu" "B.Cu") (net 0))
 (via (at 112.395 110.617) (size 0.8) (drill 0.4) (layers "F.Cu" "B.Cu") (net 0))
 (via (at 107.315 90.297) (size 0.8) (drill 0.4) (layers "F.Cu" "B.Cu") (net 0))
 (via (at 106.556 105.54) (size 0.8) (drill 0.4) (layers "F.Cu" "B.Cu") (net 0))
 (via (at 110.109 90.297) (size 0.8) (drill 0.4) (layers "F.Cu" "B.Cu") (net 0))
 (via (at 106.553 87.757) (size 0.8) (drill 0.4) (layers "F.Cu" "B.Cu") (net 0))
 (via (at 114.173 115.697) (size 0.8) (drill 0.4) (layers "F.Cu" "B.Cu") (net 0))
 (via (at 103.251 115.697) (size 0.8) (drill 0.4) (layers "F.Cu" "B.Cu") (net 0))
 (via (at 109.347 95.377) (size 0.8) (drill 0.4) (layers "F.Cu" "B.Cu") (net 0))
 (via (at 105.029 82.677) (size 0.8) (drill 0.4) (layers "F.Cu" "B.Cu") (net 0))
 (via (at 110.109 102.997) (size 0.8) (drill 0.4) (layers "F.Cu" "B.Cu") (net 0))
 (via (at 105.791 85.217) (size 0.8) (drill 0.4) (layers "F.Cu" "B.Cu") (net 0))
 (via (at 109.35 100.46) (size 0.8) (drill 0.4) (layers "F.Cu" "B.Cu") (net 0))
 (via (at 112.395 82.677) (size 0.8) (drill 0.4) (layers "F.Cu" "B.Cu") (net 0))
 (via (at 109.347 92.837) (size 0.8) (drill 0.4) (layers "F.Cu" "B.Cu") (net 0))
 (via (at 114.173 77.597) (size 0.8) (drill 0.4) (layers "F.Cu" "B.Cu") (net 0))
 (via (at 110.874 105.54) (size 0.8) (drill 0.4) (layers "F.Cu" "B.Cu") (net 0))
 (via (at 108.077 97.917) (size 0.8) (drill 0.4) (layers "F.Cu" "B.Cu") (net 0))
 (via (at 113.284 113.157) (size 0.8) (drill 0.4) (layers "F.Cu" "B.Cu") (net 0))
 (via (at 105.029 110.617) (size 0.8) (drill 0.4) (layers "F.Cu" "B.Cu") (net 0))
 (via (at 113.284 80.137) (size 0.8) (drill 0.4) (layers "F.Cu" "B.Cu") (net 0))
 (via (at 111.633 108.077) (size 0.8) (drill 0.4) (layers "F.Cu" "B.Cu") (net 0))
 (via (at 110.871 87.757) (size 0.8) (drill 0.4) (layers "F.Cu" "B.Cu") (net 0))
 (via (at 104.14 80.137) (size 0.8) (drill 0.4) (layers "F.Cu" "B.Cu") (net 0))
 (via (at 107.318 103) (size 0.8) (drill 0.4) (layers "F.Cu" "B.Cu") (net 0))
 (via (at 108.077 95.377) (size 0.8) (drill 0.4) (layers "F.Cu" "B.Cu") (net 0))
 (via (at 109.347 97.917) (size 0.8) (drill 0.4) (layers "F.Cu" "B.Cu") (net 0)))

